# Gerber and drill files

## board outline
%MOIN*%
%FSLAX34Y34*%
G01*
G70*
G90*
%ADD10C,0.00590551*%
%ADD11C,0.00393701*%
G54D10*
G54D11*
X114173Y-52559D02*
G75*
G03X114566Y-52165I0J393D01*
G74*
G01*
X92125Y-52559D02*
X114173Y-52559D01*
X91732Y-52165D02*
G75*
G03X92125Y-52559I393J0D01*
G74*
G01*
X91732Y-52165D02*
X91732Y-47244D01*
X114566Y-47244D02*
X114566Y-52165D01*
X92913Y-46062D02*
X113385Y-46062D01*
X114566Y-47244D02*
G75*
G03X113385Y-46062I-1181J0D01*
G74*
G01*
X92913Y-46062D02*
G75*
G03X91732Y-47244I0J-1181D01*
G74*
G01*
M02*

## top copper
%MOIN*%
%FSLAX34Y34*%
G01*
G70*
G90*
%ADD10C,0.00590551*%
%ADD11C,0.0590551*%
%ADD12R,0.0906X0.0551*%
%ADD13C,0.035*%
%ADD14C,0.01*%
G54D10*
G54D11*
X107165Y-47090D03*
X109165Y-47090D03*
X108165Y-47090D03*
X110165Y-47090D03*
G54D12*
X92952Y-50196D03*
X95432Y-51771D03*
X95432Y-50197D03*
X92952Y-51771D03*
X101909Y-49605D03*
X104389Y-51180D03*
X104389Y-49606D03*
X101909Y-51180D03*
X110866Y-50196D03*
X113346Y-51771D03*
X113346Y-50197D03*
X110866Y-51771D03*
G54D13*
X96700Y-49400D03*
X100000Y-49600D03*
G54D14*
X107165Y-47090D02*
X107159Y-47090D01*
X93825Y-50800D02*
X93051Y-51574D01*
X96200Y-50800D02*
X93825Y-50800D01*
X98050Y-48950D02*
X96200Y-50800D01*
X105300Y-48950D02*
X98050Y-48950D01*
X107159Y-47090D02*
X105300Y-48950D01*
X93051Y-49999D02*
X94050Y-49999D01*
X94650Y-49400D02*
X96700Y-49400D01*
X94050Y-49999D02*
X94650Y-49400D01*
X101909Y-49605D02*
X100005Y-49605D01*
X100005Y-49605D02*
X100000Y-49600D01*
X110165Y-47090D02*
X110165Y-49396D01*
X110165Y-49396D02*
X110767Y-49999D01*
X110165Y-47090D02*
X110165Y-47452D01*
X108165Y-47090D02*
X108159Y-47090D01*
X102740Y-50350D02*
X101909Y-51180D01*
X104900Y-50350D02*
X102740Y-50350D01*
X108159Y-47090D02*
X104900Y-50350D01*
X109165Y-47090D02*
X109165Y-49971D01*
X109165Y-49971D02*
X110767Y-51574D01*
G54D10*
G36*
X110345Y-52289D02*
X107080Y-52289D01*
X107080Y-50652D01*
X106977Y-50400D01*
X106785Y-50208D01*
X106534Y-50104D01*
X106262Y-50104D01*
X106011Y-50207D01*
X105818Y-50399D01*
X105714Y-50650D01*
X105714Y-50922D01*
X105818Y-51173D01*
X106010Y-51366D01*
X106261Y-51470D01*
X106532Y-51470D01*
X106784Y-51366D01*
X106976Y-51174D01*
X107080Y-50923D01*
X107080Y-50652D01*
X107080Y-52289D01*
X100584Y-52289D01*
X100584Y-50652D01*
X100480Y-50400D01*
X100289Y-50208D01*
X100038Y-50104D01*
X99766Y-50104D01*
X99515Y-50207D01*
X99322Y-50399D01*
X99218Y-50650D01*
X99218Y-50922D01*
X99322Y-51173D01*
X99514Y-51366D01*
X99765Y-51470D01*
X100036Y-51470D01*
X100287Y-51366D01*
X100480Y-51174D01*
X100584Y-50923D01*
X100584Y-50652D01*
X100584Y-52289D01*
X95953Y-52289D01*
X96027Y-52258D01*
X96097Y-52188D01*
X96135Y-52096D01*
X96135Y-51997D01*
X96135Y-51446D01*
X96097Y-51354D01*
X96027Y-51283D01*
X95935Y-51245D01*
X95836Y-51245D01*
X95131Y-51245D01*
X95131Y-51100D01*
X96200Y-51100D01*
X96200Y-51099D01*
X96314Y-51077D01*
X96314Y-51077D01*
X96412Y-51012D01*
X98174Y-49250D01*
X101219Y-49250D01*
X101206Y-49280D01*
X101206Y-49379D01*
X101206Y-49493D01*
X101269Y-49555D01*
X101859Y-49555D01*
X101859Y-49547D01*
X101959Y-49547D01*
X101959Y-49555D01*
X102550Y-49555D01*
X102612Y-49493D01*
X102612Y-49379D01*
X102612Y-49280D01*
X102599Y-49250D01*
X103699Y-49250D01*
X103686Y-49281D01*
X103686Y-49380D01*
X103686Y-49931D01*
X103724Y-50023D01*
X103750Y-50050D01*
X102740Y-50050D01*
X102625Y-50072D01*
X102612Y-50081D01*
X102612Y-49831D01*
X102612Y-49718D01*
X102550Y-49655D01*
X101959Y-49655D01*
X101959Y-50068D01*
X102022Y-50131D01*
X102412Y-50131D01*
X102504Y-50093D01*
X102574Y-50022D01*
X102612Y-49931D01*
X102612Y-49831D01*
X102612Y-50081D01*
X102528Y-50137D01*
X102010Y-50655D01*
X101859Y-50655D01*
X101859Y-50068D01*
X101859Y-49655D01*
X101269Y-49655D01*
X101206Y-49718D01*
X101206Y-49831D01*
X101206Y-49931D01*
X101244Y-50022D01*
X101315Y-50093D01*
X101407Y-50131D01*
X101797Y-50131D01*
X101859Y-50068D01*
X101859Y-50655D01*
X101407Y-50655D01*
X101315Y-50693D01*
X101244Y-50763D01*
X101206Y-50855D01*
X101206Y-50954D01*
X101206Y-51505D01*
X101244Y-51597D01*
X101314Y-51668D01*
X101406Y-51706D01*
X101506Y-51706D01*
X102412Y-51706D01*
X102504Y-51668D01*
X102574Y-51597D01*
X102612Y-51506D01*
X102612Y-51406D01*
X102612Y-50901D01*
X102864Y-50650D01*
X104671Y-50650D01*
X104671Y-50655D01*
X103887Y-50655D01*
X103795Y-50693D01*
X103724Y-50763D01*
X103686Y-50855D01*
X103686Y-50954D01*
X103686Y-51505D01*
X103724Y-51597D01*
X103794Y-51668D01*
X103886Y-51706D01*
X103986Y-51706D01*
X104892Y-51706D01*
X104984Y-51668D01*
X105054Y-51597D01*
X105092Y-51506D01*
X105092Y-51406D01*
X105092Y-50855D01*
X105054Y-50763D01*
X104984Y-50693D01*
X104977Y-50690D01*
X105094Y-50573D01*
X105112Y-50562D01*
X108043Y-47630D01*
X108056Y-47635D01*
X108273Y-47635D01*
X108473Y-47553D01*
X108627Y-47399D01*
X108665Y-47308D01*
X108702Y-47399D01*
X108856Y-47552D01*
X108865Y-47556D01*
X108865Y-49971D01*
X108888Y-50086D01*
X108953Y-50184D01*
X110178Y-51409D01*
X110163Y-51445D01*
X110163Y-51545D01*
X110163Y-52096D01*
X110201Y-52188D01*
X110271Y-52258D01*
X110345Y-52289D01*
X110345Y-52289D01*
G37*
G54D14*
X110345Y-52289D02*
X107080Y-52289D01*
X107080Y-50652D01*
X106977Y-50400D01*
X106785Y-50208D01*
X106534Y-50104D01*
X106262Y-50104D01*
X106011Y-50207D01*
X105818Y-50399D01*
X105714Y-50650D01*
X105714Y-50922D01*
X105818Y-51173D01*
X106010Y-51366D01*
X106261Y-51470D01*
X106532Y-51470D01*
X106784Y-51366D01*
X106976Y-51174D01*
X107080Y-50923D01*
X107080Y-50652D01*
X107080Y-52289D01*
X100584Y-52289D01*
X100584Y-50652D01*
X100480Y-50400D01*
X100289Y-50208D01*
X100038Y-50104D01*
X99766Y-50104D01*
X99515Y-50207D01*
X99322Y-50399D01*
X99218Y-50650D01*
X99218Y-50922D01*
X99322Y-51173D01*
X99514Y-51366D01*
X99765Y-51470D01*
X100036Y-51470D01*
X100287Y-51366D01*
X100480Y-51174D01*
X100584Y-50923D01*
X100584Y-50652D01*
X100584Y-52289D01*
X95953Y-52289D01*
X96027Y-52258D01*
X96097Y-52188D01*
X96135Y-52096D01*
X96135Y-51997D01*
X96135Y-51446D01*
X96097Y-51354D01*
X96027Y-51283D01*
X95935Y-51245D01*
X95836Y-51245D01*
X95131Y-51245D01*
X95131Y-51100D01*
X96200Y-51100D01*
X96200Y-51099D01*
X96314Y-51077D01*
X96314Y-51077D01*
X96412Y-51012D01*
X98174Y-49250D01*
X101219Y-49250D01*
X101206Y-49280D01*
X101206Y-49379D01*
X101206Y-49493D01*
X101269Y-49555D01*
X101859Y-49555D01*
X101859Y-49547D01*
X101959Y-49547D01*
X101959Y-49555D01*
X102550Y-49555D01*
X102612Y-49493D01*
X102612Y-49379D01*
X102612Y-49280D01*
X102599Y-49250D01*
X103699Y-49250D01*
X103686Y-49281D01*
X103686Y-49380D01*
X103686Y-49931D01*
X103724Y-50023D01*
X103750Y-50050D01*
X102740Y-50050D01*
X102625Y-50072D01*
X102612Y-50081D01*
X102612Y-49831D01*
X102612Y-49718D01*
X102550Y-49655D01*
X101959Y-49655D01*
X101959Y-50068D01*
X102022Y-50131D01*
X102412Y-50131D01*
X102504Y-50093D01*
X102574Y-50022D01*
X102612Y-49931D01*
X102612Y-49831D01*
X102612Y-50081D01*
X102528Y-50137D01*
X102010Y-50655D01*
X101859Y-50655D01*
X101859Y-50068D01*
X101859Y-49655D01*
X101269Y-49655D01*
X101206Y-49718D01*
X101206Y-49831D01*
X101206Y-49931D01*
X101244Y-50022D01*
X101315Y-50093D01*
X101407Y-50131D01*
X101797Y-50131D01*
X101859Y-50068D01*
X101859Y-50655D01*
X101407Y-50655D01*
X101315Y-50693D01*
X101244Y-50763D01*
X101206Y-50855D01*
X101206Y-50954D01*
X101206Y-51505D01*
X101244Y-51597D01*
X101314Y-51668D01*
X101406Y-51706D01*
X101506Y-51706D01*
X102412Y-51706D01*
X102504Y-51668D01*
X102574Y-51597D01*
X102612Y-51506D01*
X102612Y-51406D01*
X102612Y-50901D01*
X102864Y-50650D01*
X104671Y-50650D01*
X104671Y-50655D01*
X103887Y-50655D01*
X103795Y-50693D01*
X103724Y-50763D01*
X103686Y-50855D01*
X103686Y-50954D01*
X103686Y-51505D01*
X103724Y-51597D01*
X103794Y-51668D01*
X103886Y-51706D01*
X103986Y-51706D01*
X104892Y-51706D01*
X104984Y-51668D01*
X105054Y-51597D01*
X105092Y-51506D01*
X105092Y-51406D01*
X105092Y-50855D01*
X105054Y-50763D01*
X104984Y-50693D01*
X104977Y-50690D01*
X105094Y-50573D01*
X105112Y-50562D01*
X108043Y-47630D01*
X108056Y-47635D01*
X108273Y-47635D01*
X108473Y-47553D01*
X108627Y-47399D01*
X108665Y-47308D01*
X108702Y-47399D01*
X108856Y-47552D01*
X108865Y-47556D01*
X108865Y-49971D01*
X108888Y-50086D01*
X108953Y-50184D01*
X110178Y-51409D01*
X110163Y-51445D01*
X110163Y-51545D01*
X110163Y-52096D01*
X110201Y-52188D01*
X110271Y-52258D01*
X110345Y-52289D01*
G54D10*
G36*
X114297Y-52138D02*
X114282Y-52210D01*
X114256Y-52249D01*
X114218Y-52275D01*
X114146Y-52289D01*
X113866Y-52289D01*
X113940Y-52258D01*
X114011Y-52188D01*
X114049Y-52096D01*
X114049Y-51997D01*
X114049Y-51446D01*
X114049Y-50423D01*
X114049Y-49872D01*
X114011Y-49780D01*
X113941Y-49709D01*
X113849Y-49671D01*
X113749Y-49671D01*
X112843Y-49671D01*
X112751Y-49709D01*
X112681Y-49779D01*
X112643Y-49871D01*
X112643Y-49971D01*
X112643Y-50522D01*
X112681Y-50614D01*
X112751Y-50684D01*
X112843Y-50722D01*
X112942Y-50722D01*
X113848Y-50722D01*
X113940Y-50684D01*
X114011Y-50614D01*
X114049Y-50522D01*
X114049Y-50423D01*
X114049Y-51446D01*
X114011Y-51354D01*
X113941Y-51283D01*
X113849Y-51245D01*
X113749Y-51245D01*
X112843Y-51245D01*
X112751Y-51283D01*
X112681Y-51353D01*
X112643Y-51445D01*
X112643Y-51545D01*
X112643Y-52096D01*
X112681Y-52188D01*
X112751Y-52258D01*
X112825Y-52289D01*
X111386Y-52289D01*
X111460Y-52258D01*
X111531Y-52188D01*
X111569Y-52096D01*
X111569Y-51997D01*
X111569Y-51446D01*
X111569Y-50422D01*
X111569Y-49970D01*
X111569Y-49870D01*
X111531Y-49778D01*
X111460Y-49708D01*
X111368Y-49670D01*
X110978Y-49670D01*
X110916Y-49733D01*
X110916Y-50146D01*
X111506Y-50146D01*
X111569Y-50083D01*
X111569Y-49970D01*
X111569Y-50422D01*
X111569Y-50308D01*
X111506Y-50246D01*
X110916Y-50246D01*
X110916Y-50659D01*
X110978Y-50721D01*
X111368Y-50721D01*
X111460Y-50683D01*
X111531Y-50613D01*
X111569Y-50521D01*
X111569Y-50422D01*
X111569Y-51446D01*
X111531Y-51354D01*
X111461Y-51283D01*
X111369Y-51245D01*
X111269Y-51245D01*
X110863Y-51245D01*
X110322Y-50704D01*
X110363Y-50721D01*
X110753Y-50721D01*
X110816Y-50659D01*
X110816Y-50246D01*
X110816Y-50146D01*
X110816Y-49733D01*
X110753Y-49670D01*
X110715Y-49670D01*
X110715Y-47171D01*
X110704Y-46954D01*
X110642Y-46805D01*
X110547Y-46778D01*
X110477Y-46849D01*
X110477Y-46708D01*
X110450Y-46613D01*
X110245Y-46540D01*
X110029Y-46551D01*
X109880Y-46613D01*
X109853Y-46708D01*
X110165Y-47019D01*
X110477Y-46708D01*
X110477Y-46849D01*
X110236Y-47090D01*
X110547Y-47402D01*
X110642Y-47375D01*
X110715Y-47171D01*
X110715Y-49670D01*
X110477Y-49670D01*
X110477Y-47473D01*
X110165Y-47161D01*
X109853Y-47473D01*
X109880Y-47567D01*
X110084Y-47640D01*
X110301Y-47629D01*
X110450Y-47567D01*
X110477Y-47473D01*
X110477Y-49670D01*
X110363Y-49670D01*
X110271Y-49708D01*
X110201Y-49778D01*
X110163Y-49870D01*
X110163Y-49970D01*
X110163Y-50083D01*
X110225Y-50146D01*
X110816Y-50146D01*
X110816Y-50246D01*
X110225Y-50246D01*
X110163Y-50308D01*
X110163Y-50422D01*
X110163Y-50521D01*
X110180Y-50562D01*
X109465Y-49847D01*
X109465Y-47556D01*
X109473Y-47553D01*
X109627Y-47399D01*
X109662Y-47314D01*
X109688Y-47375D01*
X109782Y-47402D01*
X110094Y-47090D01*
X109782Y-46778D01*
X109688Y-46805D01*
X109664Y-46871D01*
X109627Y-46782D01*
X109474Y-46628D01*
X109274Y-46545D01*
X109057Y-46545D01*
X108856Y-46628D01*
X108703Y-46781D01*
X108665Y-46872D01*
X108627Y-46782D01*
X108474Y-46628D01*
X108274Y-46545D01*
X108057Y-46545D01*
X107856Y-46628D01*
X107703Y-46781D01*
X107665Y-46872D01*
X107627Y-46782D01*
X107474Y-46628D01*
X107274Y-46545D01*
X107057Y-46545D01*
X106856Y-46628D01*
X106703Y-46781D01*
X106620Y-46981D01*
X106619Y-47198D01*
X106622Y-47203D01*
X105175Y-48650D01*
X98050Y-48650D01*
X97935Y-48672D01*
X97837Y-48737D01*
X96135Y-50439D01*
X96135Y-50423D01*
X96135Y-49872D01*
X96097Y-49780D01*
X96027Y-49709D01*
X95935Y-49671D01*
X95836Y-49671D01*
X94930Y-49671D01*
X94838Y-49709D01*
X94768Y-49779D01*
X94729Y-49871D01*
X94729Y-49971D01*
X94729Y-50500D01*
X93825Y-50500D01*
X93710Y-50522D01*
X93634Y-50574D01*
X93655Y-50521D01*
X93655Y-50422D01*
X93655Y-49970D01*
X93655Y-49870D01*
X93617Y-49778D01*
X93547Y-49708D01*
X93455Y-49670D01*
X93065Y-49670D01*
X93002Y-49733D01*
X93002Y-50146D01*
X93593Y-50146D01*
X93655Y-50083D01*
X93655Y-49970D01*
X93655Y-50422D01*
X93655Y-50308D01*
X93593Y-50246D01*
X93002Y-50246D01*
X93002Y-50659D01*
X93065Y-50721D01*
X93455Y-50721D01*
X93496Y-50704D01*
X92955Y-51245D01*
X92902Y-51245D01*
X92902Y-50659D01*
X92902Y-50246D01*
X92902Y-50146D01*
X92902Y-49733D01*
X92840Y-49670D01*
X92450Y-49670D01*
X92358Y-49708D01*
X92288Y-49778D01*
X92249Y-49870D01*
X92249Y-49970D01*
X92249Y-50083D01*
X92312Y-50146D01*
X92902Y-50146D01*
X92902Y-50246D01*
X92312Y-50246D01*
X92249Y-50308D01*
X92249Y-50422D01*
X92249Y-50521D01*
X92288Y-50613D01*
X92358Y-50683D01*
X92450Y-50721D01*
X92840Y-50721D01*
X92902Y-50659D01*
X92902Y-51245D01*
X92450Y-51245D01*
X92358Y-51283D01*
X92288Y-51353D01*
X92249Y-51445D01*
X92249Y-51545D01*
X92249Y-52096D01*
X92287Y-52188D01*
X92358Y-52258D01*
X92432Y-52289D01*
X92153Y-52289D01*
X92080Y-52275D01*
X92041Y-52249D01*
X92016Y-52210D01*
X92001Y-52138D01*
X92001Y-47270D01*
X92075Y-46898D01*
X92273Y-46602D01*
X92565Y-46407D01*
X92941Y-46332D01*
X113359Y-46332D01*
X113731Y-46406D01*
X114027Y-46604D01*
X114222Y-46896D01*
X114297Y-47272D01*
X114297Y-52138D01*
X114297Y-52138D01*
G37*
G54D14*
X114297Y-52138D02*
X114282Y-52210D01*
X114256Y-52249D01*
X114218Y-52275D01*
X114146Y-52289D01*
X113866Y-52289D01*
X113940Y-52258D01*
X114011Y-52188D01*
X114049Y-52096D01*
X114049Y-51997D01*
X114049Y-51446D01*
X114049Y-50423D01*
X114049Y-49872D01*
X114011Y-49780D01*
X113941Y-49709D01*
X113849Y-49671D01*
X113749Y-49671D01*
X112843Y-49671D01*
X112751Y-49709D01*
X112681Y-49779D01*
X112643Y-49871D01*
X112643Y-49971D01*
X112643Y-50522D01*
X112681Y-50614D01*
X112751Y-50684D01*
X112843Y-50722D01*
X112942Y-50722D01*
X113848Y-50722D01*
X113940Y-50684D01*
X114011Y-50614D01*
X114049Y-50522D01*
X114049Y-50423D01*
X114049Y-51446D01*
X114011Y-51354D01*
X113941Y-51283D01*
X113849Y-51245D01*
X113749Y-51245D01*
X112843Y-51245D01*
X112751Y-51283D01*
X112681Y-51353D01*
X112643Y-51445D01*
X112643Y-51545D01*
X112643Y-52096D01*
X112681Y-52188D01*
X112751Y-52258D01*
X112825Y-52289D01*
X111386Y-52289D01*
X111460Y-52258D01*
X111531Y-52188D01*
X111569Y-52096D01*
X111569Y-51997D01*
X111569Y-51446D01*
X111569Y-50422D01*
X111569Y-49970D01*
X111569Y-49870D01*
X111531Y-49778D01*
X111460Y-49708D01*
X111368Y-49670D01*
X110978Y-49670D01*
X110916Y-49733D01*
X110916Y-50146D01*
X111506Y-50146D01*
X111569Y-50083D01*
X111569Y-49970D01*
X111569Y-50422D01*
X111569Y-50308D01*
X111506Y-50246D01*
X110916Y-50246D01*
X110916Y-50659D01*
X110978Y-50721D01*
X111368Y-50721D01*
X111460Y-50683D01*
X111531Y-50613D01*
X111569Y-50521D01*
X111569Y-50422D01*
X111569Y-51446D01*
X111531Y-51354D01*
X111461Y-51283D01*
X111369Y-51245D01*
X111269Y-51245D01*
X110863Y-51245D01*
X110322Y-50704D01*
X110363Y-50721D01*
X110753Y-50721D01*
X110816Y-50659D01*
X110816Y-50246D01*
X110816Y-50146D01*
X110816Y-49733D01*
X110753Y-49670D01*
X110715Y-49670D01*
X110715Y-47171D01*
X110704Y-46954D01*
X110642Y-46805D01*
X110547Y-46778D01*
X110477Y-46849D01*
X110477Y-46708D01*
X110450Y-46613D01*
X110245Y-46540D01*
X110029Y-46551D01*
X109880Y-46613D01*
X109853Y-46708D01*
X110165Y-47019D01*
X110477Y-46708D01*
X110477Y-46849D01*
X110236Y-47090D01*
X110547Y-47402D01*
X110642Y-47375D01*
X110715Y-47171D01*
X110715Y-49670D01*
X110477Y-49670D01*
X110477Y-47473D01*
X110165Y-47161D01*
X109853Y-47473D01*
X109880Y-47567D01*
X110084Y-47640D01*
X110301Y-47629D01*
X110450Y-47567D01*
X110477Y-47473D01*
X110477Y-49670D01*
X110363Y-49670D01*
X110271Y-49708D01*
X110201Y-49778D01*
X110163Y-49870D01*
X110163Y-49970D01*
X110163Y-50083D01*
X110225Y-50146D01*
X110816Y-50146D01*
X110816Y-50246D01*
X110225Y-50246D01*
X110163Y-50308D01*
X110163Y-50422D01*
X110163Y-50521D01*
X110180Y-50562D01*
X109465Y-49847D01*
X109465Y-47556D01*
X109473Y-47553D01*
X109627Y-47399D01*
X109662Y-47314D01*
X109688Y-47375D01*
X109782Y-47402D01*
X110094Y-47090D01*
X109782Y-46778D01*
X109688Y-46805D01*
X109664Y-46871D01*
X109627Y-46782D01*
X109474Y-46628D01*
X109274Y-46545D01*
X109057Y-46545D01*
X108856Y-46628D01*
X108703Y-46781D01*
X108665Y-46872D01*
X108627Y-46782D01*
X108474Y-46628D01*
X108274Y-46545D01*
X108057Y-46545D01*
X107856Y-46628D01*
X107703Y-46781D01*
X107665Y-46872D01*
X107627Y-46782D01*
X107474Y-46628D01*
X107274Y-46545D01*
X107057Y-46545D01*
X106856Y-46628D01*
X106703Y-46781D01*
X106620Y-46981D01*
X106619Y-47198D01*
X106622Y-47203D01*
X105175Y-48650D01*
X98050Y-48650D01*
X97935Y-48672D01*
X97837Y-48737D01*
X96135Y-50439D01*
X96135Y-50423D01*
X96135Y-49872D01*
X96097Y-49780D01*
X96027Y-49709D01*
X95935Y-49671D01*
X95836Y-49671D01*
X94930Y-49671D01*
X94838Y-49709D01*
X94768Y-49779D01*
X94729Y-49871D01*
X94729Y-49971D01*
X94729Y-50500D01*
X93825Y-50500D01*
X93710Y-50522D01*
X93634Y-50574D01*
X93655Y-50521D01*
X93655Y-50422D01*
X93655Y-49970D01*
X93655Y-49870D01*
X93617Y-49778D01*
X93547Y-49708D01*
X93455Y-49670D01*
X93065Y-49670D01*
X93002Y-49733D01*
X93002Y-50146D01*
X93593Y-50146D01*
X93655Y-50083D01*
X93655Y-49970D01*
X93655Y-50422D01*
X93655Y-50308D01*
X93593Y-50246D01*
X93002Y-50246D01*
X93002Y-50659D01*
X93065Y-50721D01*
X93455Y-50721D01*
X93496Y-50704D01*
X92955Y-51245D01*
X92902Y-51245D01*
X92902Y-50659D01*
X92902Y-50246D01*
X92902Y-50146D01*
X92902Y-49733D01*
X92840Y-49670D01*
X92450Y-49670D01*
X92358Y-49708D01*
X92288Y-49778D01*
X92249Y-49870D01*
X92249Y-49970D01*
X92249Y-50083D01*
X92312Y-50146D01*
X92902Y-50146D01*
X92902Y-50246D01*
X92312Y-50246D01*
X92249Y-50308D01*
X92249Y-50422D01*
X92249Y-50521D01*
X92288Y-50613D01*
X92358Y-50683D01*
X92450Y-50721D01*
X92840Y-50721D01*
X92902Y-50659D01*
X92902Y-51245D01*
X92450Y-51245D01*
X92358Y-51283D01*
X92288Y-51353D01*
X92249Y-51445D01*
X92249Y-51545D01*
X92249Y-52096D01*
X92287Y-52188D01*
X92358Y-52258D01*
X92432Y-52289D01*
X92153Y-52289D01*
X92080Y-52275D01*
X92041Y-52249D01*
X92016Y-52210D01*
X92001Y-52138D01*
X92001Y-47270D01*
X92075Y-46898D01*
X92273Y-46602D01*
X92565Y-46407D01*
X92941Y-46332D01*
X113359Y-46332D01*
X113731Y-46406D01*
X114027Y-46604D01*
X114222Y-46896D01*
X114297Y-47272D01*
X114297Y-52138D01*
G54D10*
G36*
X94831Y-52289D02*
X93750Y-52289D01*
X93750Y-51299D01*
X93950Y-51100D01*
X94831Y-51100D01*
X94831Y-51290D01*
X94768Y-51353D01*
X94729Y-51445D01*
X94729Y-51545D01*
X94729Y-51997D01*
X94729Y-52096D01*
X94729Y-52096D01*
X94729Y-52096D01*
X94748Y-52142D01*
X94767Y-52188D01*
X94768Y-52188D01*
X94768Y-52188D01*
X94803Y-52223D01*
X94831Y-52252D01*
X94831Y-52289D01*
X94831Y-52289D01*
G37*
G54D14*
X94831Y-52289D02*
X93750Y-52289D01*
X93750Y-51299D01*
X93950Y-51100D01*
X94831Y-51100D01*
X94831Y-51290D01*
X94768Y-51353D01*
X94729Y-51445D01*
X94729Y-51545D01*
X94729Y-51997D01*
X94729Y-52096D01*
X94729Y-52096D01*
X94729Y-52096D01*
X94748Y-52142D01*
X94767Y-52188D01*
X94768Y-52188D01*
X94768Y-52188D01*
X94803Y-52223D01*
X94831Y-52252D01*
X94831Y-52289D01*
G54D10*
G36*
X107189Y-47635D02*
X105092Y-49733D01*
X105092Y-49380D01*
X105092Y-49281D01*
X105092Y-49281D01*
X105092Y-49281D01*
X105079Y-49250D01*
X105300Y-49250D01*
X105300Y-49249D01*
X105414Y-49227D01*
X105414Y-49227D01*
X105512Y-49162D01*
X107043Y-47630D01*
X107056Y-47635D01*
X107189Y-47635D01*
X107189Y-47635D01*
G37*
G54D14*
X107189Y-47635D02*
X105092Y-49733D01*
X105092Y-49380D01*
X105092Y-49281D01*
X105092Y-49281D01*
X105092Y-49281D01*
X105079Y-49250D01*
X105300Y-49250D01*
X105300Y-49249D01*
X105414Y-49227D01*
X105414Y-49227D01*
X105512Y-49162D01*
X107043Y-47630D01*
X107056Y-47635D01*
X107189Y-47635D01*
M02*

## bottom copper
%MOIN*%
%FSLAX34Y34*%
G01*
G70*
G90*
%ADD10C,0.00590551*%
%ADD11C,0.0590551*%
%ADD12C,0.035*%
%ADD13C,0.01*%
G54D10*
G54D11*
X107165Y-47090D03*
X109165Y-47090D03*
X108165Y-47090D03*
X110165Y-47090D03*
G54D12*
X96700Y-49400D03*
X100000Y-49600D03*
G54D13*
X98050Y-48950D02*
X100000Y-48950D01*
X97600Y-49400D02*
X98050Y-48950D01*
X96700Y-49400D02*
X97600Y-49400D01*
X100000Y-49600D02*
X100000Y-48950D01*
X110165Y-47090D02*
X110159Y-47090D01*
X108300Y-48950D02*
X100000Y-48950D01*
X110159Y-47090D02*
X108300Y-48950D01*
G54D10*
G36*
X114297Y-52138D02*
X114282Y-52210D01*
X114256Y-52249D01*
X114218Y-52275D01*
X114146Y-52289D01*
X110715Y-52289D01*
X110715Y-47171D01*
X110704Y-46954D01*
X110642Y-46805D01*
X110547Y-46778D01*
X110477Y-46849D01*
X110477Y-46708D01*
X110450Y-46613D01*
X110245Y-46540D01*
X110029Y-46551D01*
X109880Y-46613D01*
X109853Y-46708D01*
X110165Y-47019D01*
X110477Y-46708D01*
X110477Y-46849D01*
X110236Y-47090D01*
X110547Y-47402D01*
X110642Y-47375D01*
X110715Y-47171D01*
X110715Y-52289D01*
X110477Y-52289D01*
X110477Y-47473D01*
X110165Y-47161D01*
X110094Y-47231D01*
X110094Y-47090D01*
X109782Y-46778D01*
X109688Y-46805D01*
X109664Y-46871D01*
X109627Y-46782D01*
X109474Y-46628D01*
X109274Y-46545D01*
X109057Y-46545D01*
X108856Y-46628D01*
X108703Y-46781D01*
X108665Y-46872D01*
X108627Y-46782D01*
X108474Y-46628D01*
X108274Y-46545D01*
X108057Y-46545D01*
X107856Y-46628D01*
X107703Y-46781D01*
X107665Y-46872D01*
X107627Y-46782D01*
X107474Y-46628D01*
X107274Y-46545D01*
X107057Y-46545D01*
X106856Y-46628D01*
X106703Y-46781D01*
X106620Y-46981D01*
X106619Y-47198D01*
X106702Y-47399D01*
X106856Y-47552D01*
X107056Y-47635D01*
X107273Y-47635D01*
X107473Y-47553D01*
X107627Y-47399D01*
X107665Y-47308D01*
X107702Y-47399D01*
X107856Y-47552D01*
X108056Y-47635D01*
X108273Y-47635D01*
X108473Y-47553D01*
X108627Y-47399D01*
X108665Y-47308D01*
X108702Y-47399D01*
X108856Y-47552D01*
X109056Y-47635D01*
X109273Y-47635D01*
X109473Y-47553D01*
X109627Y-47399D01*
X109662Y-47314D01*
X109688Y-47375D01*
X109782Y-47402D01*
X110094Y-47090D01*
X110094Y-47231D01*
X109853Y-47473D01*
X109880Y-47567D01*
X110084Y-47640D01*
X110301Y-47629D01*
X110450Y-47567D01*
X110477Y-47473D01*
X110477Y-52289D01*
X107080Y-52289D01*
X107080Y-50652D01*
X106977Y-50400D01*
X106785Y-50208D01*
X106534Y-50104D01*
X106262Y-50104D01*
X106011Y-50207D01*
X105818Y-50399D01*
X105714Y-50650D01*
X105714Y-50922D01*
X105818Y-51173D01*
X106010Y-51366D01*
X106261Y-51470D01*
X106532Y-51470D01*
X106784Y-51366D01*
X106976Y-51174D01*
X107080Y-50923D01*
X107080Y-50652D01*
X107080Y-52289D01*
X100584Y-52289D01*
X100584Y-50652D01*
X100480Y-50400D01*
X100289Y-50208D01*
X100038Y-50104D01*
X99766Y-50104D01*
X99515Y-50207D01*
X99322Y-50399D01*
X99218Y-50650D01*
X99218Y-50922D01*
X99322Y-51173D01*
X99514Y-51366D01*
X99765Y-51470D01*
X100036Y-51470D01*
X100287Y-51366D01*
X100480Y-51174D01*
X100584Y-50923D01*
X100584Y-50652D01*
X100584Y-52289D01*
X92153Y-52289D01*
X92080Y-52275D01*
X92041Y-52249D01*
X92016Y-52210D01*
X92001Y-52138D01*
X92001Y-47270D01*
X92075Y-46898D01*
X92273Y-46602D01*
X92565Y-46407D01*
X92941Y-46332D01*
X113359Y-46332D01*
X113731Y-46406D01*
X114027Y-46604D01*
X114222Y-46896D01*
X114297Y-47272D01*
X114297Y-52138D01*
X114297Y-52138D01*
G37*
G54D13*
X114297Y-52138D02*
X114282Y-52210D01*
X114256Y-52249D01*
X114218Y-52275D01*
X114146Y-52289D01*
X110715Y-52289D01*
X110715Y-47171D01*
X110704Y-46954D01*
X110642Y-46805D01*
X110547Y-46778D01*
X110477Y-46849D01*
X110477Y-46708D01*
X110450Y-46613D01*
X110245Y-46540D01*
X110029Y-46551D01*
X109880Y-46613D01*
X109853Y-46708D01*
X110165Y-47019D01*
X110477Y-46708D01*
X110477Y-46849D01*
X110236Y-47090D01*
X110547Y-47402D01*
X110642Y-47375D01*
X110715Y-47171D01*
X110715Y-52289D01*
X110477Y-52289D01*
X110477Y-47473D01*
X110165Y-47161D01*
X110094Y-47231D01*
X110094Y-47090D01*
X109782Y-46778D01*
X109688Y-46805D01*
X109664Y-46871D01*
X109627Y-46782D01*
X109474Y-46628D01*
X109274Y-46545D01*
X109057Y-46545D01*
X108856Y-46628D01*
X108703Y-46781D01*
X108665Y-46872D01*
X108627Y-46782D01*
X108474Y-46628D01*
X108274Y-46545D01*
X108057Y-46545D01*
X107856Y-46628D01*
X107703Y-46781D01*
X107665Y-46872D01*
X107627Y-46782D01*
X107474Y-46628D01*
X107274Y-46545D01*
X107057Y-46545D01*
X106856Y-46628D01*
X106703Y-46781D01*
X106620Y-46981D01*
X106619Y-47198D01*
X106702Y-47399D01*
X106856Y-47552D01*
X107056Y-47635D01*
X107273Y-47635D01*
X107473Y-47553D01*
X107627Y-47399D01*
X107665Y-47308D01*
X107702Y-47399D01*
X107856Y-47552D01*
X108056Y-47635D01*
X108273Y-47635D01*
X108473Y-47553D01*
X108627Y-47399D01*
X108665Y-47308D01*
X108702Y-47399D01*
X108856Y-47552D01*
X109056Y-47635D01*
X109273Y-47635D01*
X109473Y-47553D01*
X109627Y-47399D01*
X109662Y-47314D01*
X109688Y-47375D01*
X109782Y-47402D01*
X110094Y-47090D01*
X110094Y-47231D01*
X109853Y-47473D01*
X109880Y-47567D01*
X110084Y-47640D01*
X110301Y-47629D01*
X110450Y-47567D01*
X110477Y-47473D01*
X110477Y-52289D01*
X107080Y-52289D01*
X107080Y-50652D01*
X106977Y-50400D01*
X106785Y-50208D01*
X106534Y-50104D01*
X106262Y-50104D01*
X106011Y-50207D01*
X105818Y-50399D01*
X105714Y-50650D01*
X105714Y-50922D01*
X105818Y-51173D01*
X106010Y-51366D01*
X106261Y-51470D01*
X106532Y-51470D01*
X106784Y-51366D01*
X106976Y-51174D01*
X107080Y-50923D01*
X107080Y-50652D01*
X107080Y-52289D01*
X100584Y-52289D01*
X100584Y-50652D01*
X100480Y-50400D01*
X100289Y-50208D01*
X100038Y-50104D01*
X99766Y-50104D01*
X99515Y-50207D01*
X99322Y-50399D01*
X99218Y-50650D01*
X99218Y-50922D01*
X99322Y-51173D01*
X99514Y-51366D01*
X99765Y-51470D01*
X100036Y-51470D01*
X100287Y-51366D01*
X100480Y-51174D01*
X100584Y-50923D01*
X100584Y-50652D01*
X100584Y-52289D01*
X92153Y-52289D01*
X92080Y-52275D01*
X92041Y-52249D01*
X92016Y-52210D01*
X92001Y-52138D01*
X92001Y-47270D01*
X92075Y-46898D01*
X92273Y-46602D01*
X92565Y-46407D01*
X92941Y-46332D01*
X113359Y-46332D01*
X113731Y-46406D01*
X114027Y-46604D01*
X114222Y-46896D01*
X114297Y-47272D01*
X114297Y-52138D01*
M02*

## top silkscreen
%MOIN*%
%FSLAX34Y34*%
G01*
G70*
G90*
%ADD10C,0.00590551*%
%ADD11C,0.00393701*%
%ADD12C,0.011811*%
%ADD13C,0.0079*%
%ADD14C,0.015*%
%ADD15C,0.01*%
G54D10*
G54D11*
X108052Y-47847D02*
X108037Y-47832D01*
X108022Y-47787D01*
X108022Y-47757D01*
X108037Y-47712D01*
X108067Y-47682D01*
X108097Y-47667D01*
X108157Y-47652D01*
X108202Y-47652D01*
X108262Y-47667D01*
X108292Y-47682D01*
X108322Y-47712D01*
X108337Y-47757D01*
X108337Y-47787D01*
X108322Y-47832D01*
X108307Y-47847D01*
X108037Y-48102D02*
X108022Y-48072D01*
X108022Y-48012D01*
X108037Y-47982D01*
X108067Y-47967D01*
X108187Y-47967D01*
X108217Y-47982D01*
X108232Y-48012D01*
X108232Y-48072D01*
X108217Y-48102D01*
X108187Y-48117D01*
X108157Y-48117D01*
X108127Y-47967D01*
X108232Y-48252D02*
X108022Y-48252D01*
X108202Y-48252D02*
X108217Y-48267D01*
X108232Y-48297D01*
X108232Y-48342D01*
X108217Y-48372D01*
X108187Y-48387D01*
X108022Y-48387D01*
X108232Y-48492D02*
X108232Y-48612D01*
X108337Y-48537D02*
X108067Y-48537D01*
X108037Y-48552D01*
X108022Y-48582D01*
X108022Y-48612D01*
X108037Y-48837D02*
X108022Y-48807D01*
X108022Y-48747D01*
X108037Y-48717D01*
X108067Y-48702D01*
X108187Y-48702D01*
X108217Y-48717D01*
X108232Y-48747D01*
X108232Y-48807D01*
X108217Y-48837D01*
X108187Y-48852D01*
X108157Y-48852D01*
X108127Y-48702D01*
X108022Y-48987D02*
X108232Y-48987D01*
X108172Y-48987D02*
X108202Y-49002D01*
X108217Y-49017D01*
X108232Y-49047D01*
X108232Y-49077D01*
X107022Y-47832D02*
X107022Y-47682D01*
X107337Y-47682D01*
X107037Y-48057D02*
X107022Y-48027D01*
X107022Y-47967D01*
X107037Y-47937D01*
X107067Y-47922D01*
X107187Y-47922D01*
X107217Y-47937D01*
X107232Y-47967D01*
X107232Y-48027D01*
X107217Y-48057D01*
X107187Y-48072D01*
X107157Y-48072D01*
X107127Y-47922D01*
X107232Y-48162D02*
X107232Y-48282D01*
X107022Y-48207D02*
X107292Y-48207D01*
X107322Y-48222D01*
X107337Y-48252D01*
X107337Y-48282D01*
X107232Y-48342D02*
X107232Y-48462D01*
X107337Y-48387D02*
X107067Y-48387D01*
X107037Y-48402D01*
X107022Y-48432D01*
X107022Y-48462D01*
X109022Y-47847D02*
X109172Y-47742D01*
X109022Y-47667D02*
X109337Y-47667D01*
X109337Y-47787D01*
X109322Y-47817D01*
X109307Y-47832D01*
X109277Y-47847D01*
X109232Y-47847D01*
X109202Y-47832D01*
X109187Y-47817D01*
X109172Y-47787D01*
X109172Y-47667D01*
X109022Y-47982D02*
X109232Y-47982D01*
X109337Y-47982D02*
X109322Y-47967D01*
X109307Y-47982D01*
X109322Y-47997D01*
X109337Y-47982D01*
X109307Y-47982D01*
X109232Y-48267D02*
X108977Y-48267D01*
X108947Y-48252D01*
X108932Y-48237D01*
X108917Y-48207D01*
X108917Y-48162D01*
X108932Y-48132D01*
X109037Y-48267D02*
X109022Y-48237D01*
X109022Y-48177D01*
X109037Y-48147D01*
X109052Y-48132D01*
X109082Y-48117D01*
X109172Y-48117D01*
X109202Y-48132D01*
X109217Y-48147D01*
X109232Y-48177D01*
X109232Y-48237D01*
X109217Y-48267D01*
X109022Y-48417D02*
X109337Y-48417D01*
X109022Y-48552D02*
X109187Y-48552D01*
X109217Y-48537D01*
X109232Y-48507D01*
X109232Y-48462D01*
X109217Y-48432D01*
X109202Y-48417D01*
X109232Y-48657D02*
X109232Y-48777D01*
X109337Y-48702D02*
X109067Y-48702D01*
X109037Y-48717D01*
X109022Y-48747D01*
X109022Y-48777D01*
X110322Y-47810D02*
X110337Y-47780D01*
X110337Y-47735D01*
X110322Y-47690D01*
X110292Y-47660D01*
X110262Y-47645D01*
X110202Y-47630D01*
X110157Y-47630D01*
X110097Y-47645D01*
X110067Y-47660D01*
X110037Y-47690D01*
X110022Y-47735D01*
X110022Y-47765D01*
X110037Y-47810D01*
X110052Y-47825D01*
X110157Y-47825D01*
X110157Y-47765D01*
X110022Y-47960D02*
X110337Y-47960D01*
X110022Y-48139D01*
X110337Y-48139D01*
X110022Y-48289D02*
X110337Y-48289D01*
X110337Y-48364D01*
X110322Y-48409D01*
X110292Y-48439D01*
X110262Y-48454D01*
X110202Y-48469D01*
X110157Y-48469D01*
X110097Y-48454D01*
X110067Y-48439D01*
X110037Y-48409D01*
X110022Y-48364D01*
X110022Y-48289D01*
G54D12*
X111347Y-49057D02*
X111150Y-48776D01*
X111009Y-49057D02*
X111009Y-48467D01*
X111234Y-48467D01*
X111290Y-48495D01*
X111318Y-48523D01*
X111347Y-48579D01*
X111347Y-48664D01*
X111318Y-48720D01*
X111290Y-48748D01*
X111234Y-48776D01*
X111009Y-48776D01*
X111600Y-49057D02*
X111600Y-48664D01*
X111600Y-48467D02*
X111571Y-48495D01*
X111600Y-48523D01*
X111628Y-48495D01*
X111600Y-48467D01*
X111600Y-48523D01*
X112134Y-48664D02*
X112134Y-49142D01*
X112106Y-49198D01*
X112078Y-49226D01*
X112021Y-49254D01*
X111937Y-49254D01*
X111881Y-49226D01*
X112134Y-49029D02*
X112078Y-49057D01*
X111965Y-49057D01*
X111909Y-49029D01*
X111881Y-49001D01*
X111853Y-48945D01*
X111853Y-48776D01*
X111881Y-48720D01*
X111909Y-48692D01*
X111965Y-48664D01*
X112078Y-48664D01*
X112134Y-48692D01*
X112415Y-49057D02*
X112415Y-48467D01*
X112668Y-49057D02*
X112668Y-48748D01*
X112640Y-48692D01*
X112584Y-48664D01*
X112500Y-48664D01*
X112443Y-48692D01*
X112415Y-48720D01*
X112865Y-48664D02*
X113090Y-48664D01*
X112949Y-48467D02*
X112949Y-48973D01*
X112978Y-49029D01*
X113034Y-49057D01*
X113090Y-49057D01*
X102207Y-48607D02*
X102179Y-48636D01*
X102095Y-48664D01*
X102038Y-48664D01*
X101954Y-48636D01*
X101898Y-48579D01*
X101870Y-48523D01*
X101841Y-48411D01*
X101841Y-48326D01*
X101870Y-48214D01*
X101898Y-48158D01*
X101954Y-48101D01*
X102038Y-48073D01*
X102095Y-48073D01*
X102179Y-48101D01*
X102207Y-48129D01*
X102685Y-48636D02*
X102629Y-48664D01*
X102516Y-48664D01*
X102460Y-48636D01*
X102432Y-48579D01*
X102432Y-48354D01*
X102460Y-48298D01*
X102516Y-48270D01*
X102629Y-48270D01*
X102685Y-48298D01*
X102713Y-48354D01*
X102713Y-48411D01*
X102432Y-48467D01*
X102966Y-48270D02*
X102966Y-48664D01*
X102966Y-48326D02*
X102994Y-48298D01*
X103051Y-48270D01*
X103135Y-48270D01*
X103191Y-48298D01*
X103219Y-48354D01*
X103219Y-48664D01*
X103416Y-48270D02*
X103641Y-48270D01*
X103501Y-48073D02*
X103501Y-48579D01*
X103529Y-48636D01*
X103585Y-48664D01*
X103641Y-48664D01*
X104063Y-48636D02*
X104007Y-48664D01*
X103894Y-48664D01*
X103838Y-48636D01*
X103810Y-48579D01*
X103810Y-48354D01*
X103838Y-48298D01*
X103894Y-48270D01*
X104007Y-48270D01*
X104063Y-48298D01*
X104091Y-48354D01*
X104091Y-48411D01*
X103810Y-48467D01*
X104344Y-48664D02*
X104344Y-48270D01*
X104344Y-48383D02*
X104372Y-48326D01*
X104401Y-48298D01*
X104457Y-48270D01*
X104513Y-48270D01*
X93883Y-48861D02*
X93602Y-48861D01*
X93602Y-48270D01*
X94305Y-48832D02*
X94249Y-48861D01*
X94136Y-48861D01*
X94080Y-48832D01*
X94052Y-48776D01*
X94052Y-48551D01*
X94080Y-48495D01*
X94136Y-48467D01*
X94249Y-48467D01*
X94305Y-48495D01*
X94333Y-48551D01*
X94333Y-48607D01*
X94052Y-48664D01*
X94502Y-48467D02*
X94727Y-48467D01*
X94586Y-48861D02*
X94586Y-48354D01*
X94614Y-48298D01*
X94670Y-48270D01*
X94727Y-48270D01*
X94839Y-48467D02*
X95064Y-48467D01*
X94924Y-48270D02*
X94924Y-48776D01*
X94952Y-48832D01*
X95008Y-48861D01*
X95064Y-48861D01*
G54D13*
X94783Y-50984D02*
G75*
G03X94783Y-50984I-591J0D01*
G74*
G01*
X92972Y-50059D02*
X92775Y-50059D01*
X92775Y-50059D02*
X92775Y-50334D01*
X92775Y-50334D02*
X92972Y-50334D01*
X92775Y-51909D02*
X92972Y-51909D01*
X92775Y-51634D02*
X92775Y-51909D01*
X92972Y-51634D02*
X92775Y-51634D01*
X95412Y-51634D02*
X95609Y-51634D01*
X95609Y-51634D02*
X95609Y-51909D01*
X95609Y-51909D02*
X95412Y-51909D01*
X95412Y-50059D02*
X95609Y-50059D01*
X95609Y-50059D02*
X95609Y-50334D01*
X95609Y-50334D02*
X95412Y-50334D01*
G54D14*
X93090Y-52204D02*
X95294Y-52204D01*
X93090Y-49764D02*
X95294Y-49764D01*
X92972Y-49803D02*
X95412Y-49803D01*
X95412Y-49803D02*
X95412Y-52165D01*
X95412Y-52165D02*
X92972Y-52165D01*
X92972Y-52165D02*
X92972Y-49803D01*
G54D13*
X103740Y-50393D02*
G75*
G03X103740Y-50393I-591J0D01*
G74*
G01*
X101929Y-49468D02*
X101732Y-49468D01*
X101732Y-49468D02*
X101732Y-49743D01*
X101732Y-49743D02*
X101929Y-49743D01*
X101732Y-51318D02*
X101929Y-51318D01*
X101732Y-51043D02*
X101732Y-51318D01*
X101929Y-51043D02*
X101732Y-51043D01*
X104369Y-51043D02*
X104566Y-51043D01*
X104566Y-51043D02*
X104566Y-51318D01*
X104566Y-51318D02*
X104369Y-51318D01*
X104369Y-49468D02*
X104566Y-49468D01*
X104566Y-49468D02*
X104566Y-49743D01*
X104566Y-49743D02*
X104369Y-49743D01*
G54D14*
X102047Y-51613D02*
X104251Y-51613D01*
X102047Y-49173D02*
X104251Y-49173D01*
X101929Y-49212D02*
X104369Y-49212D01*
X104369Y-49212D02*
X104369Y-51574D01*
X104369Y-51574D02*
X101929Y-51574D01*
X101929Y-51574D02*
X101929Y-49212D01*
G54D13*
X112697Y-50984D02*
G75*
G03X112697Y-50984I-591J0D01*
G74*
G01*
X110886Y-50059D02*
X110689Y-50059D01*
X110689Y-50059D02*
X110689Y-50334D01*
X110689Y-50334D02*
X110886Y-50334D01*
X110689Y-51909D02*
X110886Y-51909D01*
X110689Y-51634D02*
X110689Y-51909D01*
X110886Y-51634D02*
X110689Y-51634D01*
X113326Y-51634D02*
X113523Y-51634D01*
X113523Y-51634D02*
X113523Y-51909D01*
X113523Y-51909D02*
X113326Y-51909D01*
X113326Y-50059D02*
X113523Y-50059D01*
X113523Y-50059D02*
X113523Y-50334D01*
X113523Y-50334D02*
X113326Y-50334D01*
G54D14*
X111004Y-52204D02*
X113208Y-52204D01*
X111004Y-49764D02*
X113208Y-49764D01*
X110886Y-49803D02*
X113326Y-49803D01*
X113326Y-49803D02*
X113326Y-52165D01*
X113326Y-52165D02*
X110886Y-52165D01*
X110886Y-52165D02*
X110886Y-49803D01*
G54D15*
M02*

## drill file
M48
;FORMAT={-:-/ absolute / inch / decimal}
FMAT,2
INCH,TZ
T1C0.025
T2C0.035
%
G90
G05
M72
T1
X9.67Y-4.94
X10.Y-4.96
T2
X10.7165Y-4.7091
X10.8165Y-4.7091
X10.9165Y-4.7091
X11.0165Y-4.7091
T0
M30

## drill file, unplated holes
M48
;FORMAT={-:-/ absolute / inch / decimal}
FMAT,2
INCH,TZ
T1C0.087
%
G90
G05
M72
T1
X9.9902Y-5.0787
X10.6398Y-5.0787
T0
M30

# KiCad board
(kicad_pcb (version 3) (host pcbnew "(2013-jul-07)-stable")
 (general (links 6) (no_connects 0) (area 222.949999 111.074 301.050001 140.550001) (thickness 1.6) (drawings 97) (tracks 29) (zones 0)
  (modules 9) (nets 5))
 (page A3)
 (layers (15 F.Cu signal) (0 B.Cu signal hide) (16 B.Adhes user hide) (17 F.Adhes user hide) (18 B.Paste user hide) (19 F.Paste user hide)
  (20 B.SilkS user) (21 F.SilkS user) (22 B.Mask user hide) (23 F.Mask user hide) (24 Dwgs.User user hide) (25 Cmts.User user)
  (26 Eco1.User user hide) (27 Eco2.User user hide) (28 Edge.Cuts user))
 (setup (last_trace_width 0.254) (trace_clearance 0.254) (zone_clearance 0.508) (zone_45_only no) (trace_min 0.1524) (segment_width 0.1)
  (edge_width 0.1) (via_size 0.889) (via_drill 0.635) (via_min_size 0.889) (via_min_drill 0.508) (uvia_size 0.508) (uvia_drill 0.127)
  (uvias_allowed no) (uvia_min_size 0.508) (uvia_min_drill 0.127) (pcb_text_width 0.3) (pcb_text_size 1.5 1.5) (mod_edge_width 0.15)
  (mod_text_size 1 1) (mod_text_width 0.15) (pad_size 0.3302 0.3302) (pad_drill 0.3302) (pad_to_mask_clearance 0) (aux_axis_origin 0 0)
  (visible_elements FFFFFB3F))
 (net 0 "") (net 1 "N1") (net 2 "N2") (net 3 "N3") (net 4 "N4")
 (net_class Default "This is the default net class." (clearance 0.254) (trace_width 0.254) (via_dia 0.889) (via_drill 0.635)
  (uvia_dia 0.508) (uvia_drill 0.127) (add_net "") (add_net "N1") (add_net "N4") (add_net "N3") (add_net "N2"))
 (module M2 (layer F.Cu) (at 270.25 129) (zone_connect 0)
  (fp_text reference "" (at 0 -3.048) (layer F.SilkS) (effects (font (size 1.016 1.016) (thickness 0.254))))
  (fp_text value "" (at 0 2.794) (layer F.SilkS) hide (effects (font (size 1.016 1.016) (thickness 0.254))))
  (pad "" np_thru_hole circle (at 0 0) (size 2.2 2.2) (drill 2.2) (layers *.Cu *.Mask F.SilkS) (zone_connect 0)))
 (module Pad (layer F.Cu) (at 272.2 119.61)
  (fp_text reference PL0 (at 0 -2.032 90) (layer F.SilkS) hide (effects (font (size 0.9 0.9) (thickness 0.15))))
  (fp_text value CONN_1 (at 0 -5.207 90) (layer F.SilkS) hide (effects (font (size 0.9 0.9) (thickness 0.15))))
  (pad 1 thru_hole circle (at 0 0) (size 1.5 1.5) (drill 0.9) (layers *.Cu *.Mask F.SilkS) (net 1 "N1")))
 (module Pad (layer F.Cu) (at 277.28 119.61)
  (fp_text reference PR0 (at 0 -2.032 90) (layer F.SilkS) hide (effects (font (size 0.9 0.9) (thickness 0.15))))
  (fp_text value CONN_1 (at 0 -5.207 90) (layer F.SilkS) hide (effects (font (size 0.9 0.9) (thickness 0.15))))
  (pad 1 thru_hole circle (at 0 0) (size 1.5 1.5) (drill 0.9) (layers *.Cu *.Mask F.SilkS) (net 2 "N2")))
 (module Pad (layer F.Cu) (at 274.74 119.61)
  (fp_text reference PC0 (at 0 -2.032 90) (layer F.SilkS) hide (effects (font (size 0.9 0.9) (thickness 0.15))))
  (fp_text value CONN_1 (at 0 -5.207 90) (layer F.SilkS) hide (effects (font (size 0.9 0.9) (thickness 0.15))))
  (pad 1 thru_hole circle (at 0 0) (size 1.5 1.5) (drill 0.9) (layers *.Cu *.Mask F.SilkS) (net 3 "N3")))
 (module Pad (layer F.Cu) (at 279.82 119.61)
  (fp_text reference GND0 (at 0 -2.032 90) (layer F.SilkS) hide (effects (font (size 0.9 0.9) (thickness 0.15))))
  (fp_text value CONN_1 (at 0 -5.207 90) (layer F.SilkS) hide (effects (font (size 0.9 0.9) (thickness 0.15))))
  (pad 1 thru_hole circle (at 0 0) (size 1.5 1.5) (drill 0.9) (layers *.Cu *.Mask F.SilkS) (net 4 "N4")))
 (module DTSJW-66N (layer F.Cu) (at 239.25 129.5)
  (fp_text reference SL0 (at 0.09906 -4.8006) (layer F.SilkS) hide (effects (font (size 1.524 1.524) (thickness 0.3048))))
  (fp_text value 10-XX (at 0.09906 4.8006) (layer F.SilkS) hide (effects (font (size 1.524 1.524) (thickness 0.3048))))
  (fp_circle (center 0 0) (end 1.50114 0) (layer F.SilkS) (width 0.20066))
  (fp_line (start -3.0988 -2.3495) (end -3.59918 -2.3495) (layer F.SilkS) (width 0.20066))
  (fp_line (start -3.59918 -2.3495) (end -3.59918 -1.651) (layer F.SilkS) (width 0.20066))
  (fp_line (start -3.59918 -1.651) (end -3.0988 -1.651) (layer F.SilkS) (width 0.20066))
  (fp_line (start -3.59918 2.3495) (end -3.0988 2.3495) (layer F.SilkS) (width 0.20066))
  (fp_line (start -3.59918 1.651) (end -3.59918 2.3495) (layer F.SilkS) (width 0.20066))
  (fp_line (start -3.0988 1.651) (end -3.59918 1.651) (layer F.SilkS) (width 0.20066))
  (fp_line (start 3.0988 1.651) (end 3.59918 1.651) (layer F.SilkS) (width 0.20066))
  (fp_line (start 3.59918 1.651) (end 3.59918 2.3495) (layer F.SilkS) (width 0.20066))
  (fp_line (start 3.59918 2.3495) (end 3.0988 2.3495) (layer F.SilkS) (width 0.20066))
  (fp_line (start 3.0988 -2.3495) (end 3.59918 -2.3495) (layer F.SilkS) (width 0.20066))
  (fp_line (start 3.59918 -2.3495) (end 3.59918 -1.651) (layer F.SilkS) (width 0.20066))
  (fp_line (start 3.59918 -1.651) (end 3.0988 -1.651) (layer F.SilkS) (width 0.20066))
  (fp_line (start -2.79908 3.0988) (end 2.79908 3.0988) (layer F.SilkS) (width 0.381))
  (fp_line (start -2.79908 -3.0988) (end 2.79908 -3.0988) (layer F.SilkS) (width 0.381))
  (fp_line (start -3.0988 -2.99974) (end 3.0988 -2.99974) (layer F.SilkS) (width 0.381))
  (fp_line (start 3.0988 -2.99974) (end 3.0988 2.99974) (layer F.SilkS) (width 0.381))
  (fp_line (start 3.0988 2.99974) (end -3.0988 2.99974) (layer F.SilkS) (width 0.381))
  (fp_line (start -3.0988 2.99974) (end -3.0988 -2.99974) (layer F.SilkS) (width 0.381))
  (pad 1 smd rect (at -3.1496 -2.00152) (size 2.30124 1.39954) (layers F.Cu F.Paste F.Mask) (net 4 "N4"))
  (pad 4 smd rect (at 3.1496 1.99898) (size 2.30124 1.39954) (layers F.Cu F.Paste F.Mask))
  (pad 2 smd rect (at 3.1496 -1.99898) (size 2.30124 1.39954) (layers F.Cu F.Paste F.Mask))
  (pad 3 smd rect (at -3.1496 1.99898) (size 2.30124 1.39954) (layers F.Cu F.Paste F.Mask) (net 1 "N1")))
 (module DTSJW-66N (layer F.Cu) (at 262 128)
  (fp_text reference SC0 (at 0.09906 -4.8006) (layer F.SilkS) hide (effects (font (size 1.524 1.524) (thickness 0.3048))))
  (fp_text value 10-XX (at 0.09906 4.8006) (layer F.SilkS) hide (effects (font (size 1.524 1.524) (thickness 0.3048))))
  (fp_circle (center 0 0) (end 1.50114 0) (layer F.SilkS) (width 0.20066))
  (fp_line (start -3.0988 -2.3495) (end -3.59918 -2.3495) (layer F.SilkS) (width 0.20066))
  (fp_line (start -3.59918 -2.3495) (end -3.59918 -1.651) (layer F.SilkS) (width 0.20066))
  (fp_line (start -3.59918 -1.651) (end -3.0988 -1.651) (layer F.SilkS) (width 0.20066))
  (fp_line (start -3.59918 2.3495) (end -3.0988 2.3495) (layer F.SilkS) (width 0.20066))
  (fp_line (start -3.59918 1.651) (end -3.59918 2.3495) (layer F.SilkS) (width 0.20066))
  (fp_line (start -3.0988 1.651) (end -3.59918 1.651) (layer F.SilkS) (width 0.20066))
  (fp_line (start 3.0988 1.651) (end 3.59918 1.651) (layer F.SilkS) (width 0.20066))
  (fp_line (start 3.59918 1.651) (end 3.59918 2.3495) (layer F.SilkS) (width 0.20066))
  (fp_line (start 3.59918 2.3495) (end 3.0988 2.3495) (layer F.SilkS) (width 0.20066))
  (fp_line (start 3.0988 -2.3495) (end 3.59918 -2.3495) (layer F.SilkS) (width 0.20066))
  (fp_line (start 3.59918 -2.3495) (end 3.59918 -1.651) (layer F.SilkS) (width 0.20066))
  (fp_line (start 3.59918 -1.651) (end 3.0988 -1.651) (layer F.SilkS) (width 0.20066))
  (fp_line (start -2.79908 3.0988) (end 2.79908 3.0988) (layer F.SilkS) (width 0.381))
  (fp_line (start -2.79908 -3.0988) (end 2.79908 -3.0988) (layer F.SilkS) (width 0.381))
  (fp_line (start -3.0988 -2.99974) (end 3.0988 -2.99974) (layer F.SilkS) (width 0.381))
  (fp_line (start 3.0988 -2.99974) (end 3.0988 2.99974) (layer F.SilkS) (width 0.381))
  (fp_line (start 3.0988 2.99974) (end -3.0988 2.99974) (layer F.SilkS) (width 0.381))
  (fp_line (start -3.0988 2.99974) (end -3.0988 -2.99974) (layer F.SilkS) (width 0.381))
  (pad 1 smd rect (at -3.1496 -2.00152) (size 2.30124 1.39954) (layers F.Cu F.Paste F.Mask) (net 4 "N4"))
  (pad 4 smd rect (at 3.1496 1.99898) (size 2.30124 1.39954) (layers F.Cu F.Paste F.Mask))
  (pad 2 smd rect (at 3.1496 -1.99898) (size 2.30124 1.39954) (layers F.Cu F.Paste F.Mask))
  (pad 3 smd rect (at -3.1496 1.99898) (size 2.30124 1.39954) (layers F.Cu F.Paste F.Mask) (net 3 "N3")))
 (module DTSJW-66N (layer F.Cu) (at 284.75 129.5)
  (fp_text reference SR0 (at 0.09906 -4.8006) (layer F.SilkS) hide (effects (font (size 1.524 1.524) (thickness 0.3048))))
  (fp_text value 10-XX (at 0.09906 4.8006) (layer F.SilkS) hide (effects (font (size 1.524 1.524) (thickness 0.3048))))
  (fp_circle (center 0 0) (end 1.50114 0) (layer F.SilkS) (width 0.20066))
  (fp_line (start -3.0988 -2.3495) (end -3.59918 -2.3495) (layer F.SilkS) (width 0.20066))
  (fp_line (start -3.59918 -2.3495) (end -3.59918 -1.651) (layer F.SilkS) (width 0.20066))
  (fp_line (start -3.59918 -1.651) (end -3.0988 -1.651) (layer F.SilkS) (width 0.20066))
  (fp_line (start -3.59918 2.3495) (end -3.0988 2.3495) (layer F.SilkS) (width 0.20066))
  (fp_line (start -3.59918 1.651) (end -3.59918 2.3495) (layer F.SilkS) (width 0.20066))
  (fp_line (start -3.0988 1.651) (end -3.59918 1.651) (layer F.SilkS) (width 0.20066))
  (fp_line (start 3.0988 1.651) (end 3.59918 1.651) (layer F.SilkS) (width 0.20066))
  (fp_line (start 3.59918 1.651) (end 3.59918 2.3495) (layer F.SilkS) (width 0.20066))
  (fp_line (start 3.59918 2.3495) (end 3.0988 2.3495) (layer F.SilkS) (width 0.20066))
  (fp_line (start 3.0988 -2.3495) (end 3.59918 -2.3495) (layer F.SilkS) (width 0.20066))
  (fp_line (start 3.59918 -2.3495) (end 3.59918 -1.651) (layer F.SilkS) (width 0.20066))
  (fp_line (start 3.59918 -1.651) (end 3.0988 -1.651) (layer F.SilkS) (width 0.20066))
  (fp_line (start -2.79908 3.0988) (end 2.79908 3.0988) (layer F.SilkS) (width 0.381))
  (fp_line (start -2.79908 -3.0988) (end 2.79908 -3.0988) (layer F.SilkS) (width 0.381))
  (fp_line (start -3.0988 -2.99974) (end 3.0988 -2.99974) (layer F.SilkS) (width 0.381))
  (fp_line (start 3.0988 -2.99974) (end 3.0988 2.99974) (layer F.SilkS) (width 0.381))
  (fp_line (start 3.0988 2.99974) (end -3.0988 2.99974) (layer F.SilkS) (width 0.381))
  (fp_line (start -3.0988 2.99974) (end -3.0988 -2.99974) (layer F.SilkS) (width 0.381))
  (pad 1 smd rect (at -3.1496 -2.00152) (size 2.30124 1.39954) (layers F.Cu F.Paste F.Mask) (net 4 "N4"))
  (pad 4 smd rect (at 3.1496 1.99898) (size 2.30124 1.39954) (layers F.Cu F.Paste F.Mask))
  (pad 2 smd rect (at 3.1496 -1.99898) (size 2.30124 1.39954) (layers F.Cu F.Paste F.Mask))
  (pad 3 smd rect (at -3.1496 1.99898) (size 2.30124 1.39954) (layers F.Cu F.Paste F.Mask) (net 2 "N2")))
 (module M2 (layer F.Cu) (at 253.75 129) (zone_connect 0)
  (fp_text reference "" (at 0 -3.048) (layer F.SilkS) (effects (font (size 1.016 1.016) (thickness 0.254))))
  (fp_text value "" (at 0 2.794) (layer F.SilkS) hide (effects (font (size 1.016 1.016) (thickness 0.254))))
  (pad "" np_thru_hole circle (at 0 0) (size 2.2 2.2) (drill 2.2) (layers *.Cu *.Mask F.SilkS) (zone_connect 0)))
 (gr_arc (start 290 132.5) (end 291 132.5) (angle 90) (layer Edge.Cuts) (width 0.1))
 (gr_line (start 234 133.5) (end 290 133.5) (angle 90) (layer Edge.Cuts) (width 0.1))
 (gr_arc (start 234 132.5) (end 234 133.5) (angle 90) (layer Edge.Cuts) (width 0.1))
 (gr_line (start 233 132.5) (end 233 120) (angle 90) (layer Edge.Cuts) (width 0.1))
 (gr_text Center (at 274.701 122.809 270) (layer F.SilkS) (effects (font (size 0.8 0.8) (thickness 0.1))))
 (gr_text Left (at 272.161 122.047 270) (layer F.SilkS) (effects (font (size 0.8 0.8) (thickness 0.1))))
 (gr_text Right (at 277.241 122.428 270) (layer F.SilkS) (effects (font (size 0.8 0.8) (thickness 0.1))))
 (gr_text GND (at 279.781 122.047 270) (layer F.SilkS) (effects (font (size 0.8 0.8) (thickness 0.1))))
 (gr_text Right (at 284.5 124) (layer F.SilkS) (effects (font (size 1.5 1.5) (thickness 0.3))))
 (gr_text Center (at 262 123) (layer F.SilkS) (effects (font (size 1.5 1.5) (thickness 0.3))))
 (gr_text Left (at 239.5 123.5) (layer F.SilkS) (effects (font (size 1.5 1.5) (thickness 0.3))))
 (gr_line (start 291 120) (end 291 132.5) (angle 90) (layer Edge.Cuts) (width 0.1))
 (gr_line (start 236 117) (end 288 117) (angle 90) (layer Edge.Cuts) (width 0.1))
 (gr_arc (start 288 120) (end 288 117) (angle 90) (layer Edge.Cuts) (width 0.1))
 (gr_arc (start 236 120) (end 233 120) (angle 90) (layer Edge.Cuts) (width 0.1))
 (segment (start 272.2 119.61) (end 272.185 119.61) (width 0.254) (layer F.Cu) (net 1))
 (segment (start 238.31738 129.032) (end 236.3504 130.99898) (width 0.254) (layer F.Cu) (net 1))
 (segment (start 244.348 129.032) (end 238.31738 129.032) (width 0.254) (layer F.Cu) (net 1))
 (segment (start 249.047 124.333) (end 244.348 129.032) (width 0.254) (layer F.Cu) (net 1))
 (segment (start 267.462 124.333) (end 249.047 124.333) (width 0.254) (layer F.Cu) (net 1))
 (segment (start 272.185 119.61) (end 267.462 124.333) (width 0.254) (layer F.Cu) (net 1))
 (segment (start 236.3504 126.99848) (end 238.88852 126.99848) (width 0.254) (layer F.Cu) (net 4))
 (segment (start 249.047 124.333) (end 254 124.333) (width 0.254) (layer B.Cu) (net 4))
 (segment (start 247.904 125.476) (end 249.047 124.333) (width 0.254) (layer B.Cu) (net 4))
 (segment (start 245.618 125.476) (end 247.904 125.476) (width 0.254) (layer B.Cu) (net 4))
 (via (at 245.618 125.476) (size 0.889) (layers F.Cu B.Cu) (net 4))
 (segment (start 240.411 125.476) (end 245.618 125.476) (width 0.254) (layer F.Cu) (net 4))
 (segment (start 238.88852 126.99848) (end 240.411 125.476) (width 0.254) (layer F.Cu) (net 4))
 (segment (start 258.8504 125.99848) (end 254.01448 125.99848) (width 0.254) (layer F.Cu) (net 4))
 (segment (start 254 125.984) (end 254 124.333) (width 0.254) (layer B.Cu) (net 4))
 (via (at 254 125.984) (size 0.889) (layers F.Cu B.Cu) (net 4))
 (segment (start 254.01448 125.99848) (end 254 125.984) (width 0.254) (layer F.Cu) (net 4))
 (segment (start 279.82 119.61) (end 279.805 119.61) (width 0.254) (layer B.Cu) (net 4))
 (segment (start 275.082 124.333) (end 254 124.333) (width 0.254) (layer B.Cu) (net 4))
 (segment (start 279.805 119.61) (end 275.082 124.333) (width 0.254) (layer B.Cu) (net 4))
 (segment (start 279.82 119.61) (end 279.82 125.46808) (width 0.254) (layer F.Cu) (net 4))
 (segment (start 279.82 125.46808) (end 281.3504 126.99848) (width 0.254) (layer F.Cu) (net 4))
 (segment (start 279.82 119.61) (end 279.82 120.52888) (width 0.254) (layer F.Cu) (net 4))
 (segment (start 274.74 119.61) (end 274.725 119.61) (width 0.254) (layer F.Cu) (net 3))
 (segment (start 260.96038 127.889) (end 258.8504 129.99898) (width 0.254) (layer F.Cu) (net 3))
 (segment (start 266.446 127.889) (end 260.96038 127.889) (width 0.254) (layer F.Cu) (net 3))
 (segment (start 274.725 119.61) (end 266.446 127.889) (width 0.254) (layer F.Cu) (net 3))
 (segment (start 277.28 119.61) (end 277.28 126.92858) (width 0.254) (layer F.Cu) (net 2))
 (segment (start 277.28 126.92858) (end 281.3504 130.99898) (width 0.254) (layer F.Cu) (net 2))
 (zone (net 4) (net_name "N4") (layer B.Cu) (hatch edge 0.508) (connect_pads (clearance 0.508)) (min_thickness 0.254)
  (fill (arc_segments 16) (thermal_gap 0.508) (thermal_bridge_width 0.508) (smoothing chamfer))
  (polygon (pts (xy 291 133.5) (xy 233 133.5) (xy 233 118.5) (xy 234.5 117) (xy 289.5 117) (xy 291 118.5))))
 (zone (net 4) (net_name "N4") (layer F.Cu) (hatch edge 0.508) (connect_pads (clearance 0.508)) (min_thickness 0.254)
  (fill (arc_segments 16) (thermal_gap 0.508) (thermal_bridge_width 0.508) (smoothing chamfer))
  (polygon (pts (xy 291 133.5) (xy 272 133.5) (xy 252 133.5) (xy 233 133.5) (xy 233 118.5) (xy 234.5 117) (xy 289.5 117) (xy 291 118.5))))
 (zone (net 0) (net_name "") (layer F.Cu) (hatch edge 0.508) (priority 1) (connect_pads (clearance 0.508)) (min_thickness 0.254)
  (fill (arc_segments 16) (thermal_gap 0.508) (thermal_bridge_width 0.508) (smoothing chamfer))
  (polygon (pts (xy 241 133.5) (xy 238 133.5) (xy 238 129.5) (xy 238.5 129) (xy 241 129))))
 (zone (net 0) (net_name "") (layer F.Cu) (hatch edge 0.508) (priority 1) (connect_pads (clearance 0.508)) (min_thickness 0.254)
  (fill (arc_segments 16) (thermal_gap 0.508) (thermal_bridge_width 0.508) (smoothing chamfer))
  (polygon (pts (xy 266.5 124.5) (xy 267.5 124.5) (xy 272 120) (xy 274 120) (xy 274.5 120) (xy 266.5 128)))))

